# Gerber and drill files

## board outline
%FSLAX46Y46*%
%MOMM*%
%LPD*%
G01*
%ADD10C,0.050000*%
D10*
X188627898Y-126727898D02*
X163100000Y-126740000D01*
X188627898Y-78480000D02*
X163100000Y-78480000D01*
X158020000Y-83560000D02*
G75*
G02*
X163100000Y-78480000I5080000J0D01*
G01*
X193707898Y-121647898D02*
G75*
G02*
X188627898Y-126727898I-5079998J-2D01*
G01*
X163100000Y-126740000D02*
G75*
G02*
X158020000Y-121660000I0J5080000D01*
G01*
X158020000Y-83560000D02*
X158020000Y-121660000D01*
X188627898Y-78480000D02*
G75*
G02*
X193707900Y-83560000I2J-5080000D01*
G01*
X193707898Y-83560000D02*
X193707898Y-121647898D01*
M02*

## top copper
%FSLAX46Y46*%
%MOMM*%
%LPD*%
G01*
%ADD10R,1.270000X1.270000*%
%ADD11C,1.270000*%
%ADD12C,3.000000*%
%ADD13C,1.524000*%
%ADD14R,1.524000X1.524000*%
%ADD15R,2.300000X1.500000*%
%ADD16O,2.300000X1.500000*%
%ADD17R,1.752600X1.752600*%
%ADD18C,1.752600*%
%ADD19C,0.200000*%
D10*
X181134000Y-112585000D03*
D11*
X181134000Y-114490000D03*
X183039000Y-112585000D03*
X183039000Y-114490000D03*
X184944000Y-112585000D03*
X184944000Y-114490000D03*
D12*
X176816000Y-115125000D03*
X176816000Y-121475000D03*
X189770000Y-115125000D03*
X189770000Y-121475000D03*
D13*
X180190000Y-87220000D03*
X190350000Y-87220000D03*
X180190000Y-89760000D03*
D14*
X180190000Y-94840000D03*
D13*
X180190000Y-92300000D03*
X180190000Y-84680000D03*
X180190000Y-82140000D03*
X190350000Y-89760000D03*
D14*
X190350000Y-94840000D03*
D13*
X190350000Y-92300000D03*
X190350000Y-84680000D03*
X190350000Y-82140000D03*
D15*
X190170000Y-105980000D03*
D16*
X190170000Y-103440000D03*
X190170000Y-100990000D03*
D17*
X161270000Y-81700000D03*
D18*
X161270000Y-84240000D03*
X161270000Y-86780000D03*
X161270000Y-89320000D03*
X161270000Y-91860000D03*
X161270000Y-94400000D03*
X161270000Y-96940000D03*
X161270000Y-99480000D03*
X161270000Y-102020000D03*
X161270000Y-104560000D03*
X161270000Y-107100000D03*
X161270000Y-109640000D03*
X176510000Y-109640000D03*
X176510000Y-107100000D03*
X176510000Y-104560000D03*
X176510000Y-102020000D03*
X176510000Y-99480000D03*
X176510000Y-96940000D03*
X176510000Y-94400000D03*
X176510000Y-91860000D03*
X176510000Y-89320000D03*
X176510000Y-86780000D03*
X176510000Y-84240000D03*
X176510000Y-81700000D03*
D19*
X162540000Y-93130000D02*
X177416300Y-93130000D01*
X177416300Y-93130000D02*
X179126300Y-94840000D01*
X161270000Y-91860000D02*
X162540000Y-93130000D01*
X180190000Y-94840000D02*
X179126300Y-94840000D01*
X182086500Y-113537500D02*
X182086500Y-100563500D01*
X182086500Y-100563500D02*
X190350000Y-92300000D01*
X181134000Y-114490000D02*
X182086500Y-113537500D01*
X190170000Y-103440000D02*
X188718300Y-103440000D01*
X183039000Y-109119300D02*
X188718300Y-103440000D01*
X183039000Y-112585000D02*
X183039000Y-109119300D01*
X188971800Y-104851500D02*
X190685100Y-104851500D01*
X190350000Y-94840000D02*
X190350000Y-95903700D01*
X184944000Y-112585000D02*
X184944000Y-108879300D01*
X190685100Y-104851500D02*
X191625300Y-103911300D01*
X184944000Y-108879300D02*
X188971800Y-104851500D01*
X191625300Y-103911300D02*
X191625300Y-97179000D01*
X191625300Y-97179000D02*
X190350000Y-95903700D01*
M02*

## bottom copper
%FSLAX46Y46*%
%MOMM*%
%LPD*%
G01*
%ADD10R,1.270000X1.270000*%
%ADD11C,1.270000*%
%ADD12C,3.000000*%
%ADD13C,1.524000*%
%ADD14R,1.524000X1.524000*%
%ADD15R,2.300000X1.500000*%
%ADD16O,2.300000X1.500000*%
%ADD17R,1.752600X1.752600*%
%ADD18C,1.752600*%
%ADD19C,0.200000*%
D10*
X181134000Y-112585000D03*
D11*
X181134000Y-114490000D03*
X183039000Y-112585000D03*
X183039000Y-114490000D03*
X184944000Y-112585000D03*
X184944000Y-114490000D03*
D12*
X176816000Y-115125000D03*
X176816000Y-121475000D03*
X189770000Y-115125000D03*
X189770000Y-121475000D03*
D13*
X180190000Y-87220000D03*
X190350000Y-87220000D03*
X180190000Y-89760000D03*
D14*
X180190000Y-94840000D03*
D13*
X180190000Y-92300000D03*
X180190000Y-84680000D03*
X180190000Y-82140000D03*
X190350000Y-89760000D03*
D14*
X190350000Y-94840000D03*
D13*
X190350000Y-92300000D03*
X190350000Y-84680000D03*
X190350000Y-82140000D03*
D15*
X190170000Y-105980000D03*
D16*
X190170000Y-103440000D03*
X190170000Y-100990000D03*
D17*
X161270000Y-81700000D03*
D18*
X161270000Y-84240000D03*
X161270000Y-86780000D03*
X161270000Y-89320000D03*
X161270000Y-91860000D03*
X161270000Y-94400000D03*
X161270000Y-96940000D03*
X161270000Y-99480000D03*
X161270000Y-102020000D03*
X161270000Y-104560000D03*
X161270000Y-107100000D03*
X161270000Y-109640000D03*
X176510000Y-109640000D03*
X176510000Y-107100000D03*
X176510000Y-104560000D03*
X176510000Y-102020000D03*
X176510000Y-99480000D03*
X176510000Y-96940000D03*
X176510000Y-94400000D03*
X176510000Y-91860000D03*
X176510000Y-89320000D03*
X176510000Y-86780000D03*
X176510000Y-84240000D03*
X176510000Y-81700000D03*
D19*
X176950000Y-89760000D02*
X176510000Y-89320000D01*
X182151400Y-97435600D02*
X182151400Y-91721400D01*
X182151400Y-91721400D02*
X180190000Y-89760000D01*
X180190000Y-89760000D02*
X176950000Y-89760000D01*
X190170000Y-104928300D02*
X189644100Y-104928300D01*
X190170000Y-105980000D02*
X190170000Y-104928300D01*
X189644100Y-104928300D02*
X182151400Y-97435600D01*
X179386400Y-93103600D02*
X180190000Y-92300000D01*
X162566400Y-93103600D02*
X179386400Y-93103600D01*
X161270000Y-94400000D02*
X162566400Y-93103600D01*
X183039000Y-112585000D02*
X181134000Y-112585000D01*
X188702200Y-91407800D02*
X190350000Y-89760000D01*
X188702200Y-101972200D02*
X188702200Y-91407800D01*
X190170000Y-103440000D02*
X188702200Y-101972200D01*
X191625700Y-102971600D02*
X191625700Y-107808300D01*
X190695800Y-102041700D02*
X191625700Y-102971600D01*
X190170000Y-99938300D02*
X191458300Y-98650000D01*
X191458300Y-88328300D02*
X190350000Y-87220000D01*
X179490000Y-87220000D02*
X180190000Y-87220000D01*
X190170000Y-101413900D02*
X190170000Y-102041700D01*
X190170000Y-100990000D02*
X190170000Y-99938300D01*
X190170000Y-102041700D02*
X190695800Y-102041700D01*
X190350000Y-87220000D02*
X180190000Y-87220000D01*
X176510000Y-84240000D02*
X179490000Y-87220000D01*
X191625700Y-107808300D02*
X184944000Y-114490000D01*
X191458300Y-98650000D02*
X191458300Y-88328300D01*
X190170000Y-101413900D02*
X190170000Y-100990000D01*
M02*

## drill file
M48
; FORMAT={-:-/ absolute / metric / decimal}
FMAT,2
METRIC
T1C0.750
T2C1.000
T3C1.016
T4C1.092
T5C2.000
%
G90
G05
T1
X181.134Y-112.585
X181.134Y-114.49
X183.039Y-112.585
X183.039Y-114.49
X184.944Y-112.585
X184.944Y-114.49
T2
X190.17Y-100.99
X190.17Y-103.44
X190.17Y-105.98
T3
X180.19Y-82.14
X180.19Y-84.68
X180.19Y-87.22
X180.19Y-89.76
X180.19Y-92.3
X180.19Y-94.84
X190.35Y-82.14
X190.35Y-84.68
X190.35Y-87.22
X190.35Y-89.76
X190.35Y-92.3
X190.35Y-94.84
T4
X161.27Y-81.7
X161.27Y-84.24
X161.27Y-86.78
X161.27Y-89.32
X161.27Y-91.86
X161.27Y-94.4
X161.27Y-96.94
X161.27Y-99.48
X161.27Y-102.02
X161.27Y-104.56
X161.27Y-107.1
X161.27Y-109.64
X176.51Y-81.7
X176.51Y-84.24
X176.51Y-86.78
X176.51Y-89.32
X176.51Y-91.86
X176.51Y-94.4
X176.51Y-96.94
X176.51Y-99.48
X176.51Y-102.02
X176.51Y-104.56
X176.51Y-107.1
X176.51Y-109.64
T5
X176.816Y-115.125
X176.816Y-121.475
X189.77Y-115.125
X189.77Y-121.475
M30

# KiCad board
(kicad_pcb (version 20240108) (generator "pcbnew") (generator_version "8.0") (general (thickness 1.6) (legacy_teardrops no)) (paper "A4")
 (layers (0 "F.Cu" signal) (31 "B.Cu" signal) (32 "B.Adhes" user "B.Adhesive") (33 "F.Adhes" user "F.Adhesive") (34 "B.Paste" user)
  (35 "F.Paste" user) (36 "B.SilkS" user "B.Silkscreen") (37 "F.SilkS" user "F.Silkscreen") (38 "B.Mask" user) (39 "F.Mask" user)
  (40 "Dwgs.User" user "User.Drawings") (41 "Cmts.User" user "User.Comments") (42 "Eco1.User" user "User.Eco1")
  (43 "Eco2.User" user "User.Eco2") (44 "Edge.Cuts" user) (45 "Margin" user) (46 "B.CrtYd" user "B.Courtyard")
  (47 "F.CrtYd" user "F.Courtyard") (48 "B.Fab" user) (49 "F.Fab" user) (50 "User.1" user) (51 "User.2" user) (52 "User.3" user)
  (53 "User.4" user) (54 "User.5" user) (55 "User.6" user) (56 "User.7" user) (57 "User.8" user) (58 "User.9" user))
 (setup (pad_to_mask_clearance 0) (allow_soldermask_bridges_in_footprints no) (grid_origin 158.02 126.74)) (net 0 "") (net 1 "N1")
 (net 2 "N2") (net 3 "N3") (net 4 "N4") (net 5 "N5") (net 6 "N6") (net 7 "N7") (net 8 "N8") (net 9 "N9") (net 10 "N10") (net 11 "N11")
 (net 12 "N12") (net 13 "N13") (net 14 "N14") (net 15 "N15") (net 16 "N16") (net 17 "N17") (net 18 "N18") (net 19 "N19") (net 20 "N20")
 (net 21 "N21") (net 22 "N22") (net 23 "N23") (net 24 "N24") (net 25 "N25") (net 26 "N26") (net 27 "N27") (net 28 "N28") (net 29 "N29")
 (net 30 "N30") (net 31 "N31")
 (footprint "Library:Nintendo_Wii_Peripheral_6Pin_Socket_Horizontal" (layer "F.Cu") (at 181.134 112.585)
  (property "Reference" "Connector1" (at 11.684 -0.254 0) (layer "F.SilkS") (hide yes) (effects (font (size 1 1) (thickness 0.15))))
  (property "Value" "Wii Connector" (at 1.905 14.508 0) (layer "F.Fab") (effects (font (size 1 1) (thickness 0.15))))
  (pad "1" thru_hole rect (at 0 0 180) (size 1.27 1.27) (drill 0.75) (layers "*.Cu" "*.Mask") (remove_unused_layers no) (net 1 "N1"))
  (pad "2" thru_hole circle (at 0 1.905 180) (size 1.27 1.27) (drill 0.75) (layers "*.Cu" "*.Mask") (remove_unused_layers no) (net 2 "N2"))
  (pad "3" thru_hole circle (at 1.905 0 180) (size 1.27 1.27) (drill 0.75) (layers "*.Cu" "*.Mask") (remove_unused_layers no) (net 1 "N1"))
  (pad "4" thru_hole circle (at 1.905 1.905 180) (size 1.27 1.27) (drill 0.75) (layers "*.Cu" "*.Mask") (remove_unused_layers no))
  (pad "5" thru_hole circle (at 3.81 0 180) (size 1.27 1.27) (drill 0.75) (layers "*.Cu" "*.Mask") (remove_unused_layers no) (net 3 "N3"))
  (pad "6" thru_hole circle (at 3.81 1.905 180) (size 1.27 1.27) (drill 0.75) (layers "*.Cu" "*.Mask") (remove_unused_layers no)
   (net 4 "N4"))
  (pad "SH" thru_hole circle (at -4.318 2.54 180) (size 3 3) (drill 2) (layers "*.Cu" "*.Mask") (remove_unused_layers no))
  (pad "SH" thru_hole circle (at -4.318 8.89 180) (size 3 3) (drill 2) (layers "*.Cu" "*.Mask") (remove_unused_layers no))
  (pad "SH" thru_hole circle (at 8.636 2.54 180) (size 3 3) (drill 2) (layers "*.Cu" "*.Mask") (remove_unused_layers no))
  (pad "SH" thru_hole circle (at 8.636 8.89 180) (size 3 3) (drill 2) (layers "*.Cu" "*.Mask") (remove_unused_layers no))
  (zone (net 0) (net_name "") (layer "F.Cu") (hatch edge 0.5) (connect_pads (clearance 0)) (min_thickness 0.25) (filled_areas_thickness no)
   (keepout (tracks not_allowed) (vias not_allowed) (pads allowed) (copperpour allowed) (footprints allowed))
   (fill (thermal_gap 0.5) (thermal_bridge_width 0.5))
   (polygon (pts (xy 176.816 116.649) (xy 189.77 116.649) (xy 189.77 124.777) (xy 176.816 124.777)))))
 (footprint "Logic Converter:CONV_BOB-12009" (layer "F.Cu") (at 185.27 88.49 180)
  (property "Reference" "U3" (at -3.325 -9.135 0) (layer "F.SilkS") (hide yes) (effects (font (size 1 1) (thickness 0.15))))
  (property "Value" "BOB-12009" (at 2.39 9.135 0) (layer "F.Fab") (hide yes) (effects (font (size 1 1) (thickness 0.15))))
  (pad "GND_1" thru_hole circle (at 5.08 1.27 180) (size 1.524 1.524) (drill 1.016) (layers "*.Cu" "*.Mask") (remove_unused_layers no)
   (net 4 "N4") (solder_mask_margin 0.102))
  (pad "GND_2" thru_hole circle (at -5.08 1.27 180) (size 1.524 1.524) (drill 1.016) (layers "*.Cu" "*.Mask") (remove_unused_layers no)
   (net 4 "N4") (solder_mask_margin 0.102))
  (pad "HV" thru_hole circle (at 5.08 -1.27 180) (size 1.524 1.524) (drill 1.016) (layers "*.Cu" "*.Mask") (remove_unused_layers no)
   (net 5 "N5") (solder_mask_margin 0.102))
  (pad "HV1" thru_hole rect (at 5.08 -6.35 180) (size 1.524 1.524) (drill 1.016) (layers "*.Cu" "*.Mask") (remove_unused_layers no)
   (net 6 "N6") (solder_mask_margin 0.102))
  (pad "HV2" thru_hole circle (at 5.08 -3.81 180) (size 1.524 1.524) (drill 1.016) (layers "*.Cu" "*.Mask") (remove_unused_layers no)
   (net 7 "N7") (solder_mask_margin 0.102))
  (pad "HV3" thru_hole circle (at 5.08 3.81 180) (size 1.524 1.524) (drill 1.016) (layers "*.Cu" "*.Mask") (remove_unused_layers no)
   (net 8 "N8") (solder_mask_margin 0.102))
  (pad "HV4" thru_hole circle (at 5.08 6.35 180) (size 1.524 1.524) (drill 1.016) (layers "*.Cu" "*.Mask") (remove_unused_layers no)
   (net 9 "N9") (solder_mask_margin 0.102))
  (pad "LV" thru_hole circle (at -5.08 -1.27 180) (size 1.524 1.524) (drill 1.016) (layers "*.Cu" "*.Mask") (remove_unused_layers no)
   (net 1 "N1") (solder_mask_margin 0.102))
  (pad "LV1" thru_hole rect (at -5.08 -6.35 180) (size 1.524 1.524) (drill 1.016) (layers "*.Cu" "*.Mask") (remove_unused_layers no)
   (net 3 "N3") (solder_mask_margin 0.102))
  (pad "LV2" thru_hole circle (at -5.08 -3.81 180) (size 1.524 1.524) (drill 1.016) (layers "*.Cu" "*.Mask") (remove_unused_layers no)
   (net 2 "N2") (solder_mask_margin 0.102))
  (pad "LV3" thru_hole circle (at -5.08 3.81 180) (size 1.524 1.524) (drill 1.016) (layers "*.Cu" "*.Mask") (remove_unused_layers no)
   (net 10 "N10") (solder_mask_margin 0.102))
  (pad "LV4" thru_hole circle (at -5.08 6.35 180) (size 1.524 1.524) (drill 1.016) (layers "*.Cu" "*.Mask") (remove_unused_layers no)
   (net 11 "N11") (solder_mask_margin 0.102)))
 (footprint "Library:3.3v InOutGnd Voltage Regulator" (layer "F.Cu") (at 191.67 103.49 90)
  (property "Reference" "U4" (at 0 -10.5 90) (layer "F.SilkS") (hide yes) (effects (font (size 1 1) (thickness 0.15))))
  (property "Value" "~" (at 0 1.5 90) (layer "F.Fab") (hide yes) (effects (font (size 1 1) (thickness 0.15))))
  (pad "1" thru_hole rect (at -2.49 -1.5 90) (size 1.5 2.3) (drill 1) (layers "*.Cu" "*.Mask") (remove_unused_layers no) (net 5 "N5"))
  (pad "2" thru_hole oval (at 0.05 -1.5 90) (size 1.5 2.3) (drill 1) (layers "*.Cu" "*.Mask") (remove_unused_layers no) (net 1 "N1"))
  (pad "3" thru_hole oval (at 2.5 -1.5 90) (size 1.5 2.3) (drill 1) (layers "*.Cu" "*.Mask") (remove_unused_layers no) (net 4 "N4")))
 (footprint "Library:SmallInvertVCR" (layer "F.Cu") (at 166.77 116.74)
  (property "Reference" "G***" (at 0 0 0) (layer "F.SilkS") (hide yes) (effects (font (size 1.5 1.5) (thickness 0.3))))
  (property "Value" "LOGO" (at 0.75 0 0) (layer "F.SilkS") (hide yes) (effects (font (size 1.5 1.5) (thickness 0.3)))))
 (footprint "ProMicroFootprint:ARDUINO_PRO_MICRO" (layer "F.Cu") (at 168.89 95.67 -90)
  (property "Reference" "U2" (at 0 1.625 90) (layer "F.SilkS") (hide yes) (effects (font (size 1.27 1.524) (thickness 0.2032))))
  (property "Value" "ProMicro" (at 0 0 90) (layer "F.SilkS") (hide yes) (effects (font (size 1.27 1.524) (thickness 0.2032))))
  (pad "1" thru_hole rect (at -13.97 7.62 270) (size 1.7526 1.7526) (drill 1.0922) (layers "*.Cu" "*.SilkS" "*.Mask")
   (remove_unused_layers no) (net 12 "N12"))
  (pad "2" thru_hole circle (at -11.43 7.62 270) (size 1.7526 1.7526) (drill 1.0922) (layers "*.Cu" "*.SilkS" "*.Mask")
   (remove_unused_layers no) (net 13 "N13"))
  (pad "3" thru_hole circle (at -8.89 7.62 270) (size 1.7526 1.7526) (drill 1.0922) (layers "*.Cu" "*.SilkS" "*.Mask")
   (remove_unused_layers no) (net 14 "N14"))
  (pad "4" thru_hole circle (at -6.35 7.62 270) (size 1.7526 1.7526) (drill 1.0922) (layers "*.Cu" "*.SilkS" "*.Mask")
   (remove_unused_layers no) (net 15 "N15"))
  (pad "5" thru_hole circle (at -3.81 7.62 270) (size 1.7526 1.7526) (drill 1.0922) (layers "*.Cu" "*.SilkS" "*.Mask")
   (remove_unused_layers no) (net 6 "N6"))
  (pad "6" thru_hole circle (at -1.27 7.62 270) (size 1.7526 1.7526) (drill 1.0922) (layers "*.Cu" "*.SilkS" "*.Mask")
   (remove_unused_layers no) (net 7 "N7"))
  (pad "7" thru_hole circle (at 1.27 7.62 270) (size 1.7526 1.7526) (drill 1.0922) (layers "*.Cu" "*.SilkS" "*.Mask")
   (remove_unused_layers no) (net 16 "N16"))
  (pad "8" thru_hole circle (at 3.81 7.62 270) (size 1.7526 1.7526) (drill 1.0922) (layers "*.Cu" "*.SilkS" "*.Mask")
   (remove_unused_layers no) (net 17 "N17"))
  (pad "9" thru_hole circle (at 6.35 7.62 270) (size 1.7526 1.7526) (drill 1.0922) (layers "*.Cu" "*.SilkS" "*.Mask")
   (remove_unused_layers no) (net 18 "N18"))
  (pad "10" thru_hole circle (at 8.89 7.62 270) (size 1.7526 1.7526) (drill 1.0922) (layers "*.Cu" "*.SilkS" "*.Mask")
   (remove_unused_layers no) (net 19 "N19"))
  (pad "11" thru_hole circle (at 11.43 7.62 270) (size 1.7526 1.7526) (drill 1.0922) (layers "*.Cu" "*.SilkS" "*.Mask")
   (remove_unused_layers no) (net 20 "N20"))
  (pad "12" thru_hole circle (at 13.97 7.62 270) (size 1.7526 1.7526) (drill 1.0922) (layers "*.Cu" "*.SilkS" "*.Mask")
   (remove_unused_layers no) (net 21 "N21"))
  (pad "13" thru_hole circle (at 13.97 -7.62 270) (size 1.7526 1.7526) (drill 1.0922) (layers "*.Cu" "*.SilkS" "*.Mask")
   (remove_unused_layers no) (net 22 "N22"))
  (pad "14" thru_hole circle (at 11.43 -7.62 270) (size 1.7526 1.7526) (drill 1.0922) (layers "*.Cu" "*.SilkS" "*.Mask")
   (remove_unused_layers no) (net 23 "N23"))
  (pad "15" thru_hole circle (at 8.89 -7.62 270) (size 1.7526 1.7526) (drill 1.0922) (layers "*.Cu" "*.SilkS" "*.Mask")
   (remove_unused_layers no) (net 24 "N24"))
  (pad "16" thru_hole circle (at 6.35 -7.62 270) (size 1.7526 1.7526) (drill 1.0922) (layers "*.Cu" "*.SilkS" "*.Mask")
   (remove_unused_layers no) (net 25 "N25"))
  (pad "17" thru_hole circle (at 3.81 -7.62 270) (size 1.7526 1.7526) (drill 1.0922) (layers "*.Cu" "*.SilkS" "*.Mask")
   (remove_unused_layers no) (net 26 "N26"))
  (pad "18" thru_hole circle (at 1.27 -7.62 270) (size 1.7526 1.7526) (drill 1.0922) (layers "*.Cu" "*.SilkS" "*.Mask")
   (remove_unused_layers no) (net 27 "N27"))
  (pad "19" thru_hole circle (at -1.27 -7.62 270) (size 1.7526 1.7526) (drill 1.0922) (layers "*.Cu" "*.SilkS" "*.Mask")
   (remove_unused_layers no) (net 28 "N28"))
  (pad "20" thru_hole circle (at -3.81 -7.62 270) (size 1.7526 1.7526) (drill 1.0922) (layers "*.Cu" "*.SilkS" "*.Mask")
   (remove_unused_layers no) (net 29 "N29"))
  (pad "21" thru_hole circle (at -6.35 -7.62 270) (size 1.7526 1.7526) (drill 1.0922) (layers "*.Cu" "*.SilkS" "*.Mask")
   (remove_unused_layers no) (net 5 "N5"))
  (pad "22" thru_hole circle (at -8.89 -7.62 270) (size 1.7526 1.7526) (drill 1.0922) (layers "*.Cu" "*.SilkS" "*.Mask")
   (remove_unused_layers no) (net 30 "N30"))
  (pad "23" thru_hole circle (at -11.43 -7.62 270) (size 1.7526 1.7526) (drill 1.0922) (layers "*.Cu" "*.SilkS" "*.Mask")
   (remove_unused_layers no) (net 4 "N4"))
  (pad "24" thru_hole circle (at -13.97 -7.62 270) (size 1.7526 1.7526) (drill 1.0922) (layers "*.Cu" "*.SilkS" "*.Mask")
   (remove_unused_layers no) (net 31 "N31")))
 (gr_line (start 188.627898 126.727898) (end 163.1 126.74) (stroke (width 0.05) (type default)) (layer "Edge.Cuts"))
 (gr_line (start 188.627898 78.48) (end 163.1 78.48) (stroke (width 0.05) (type default)) (layer "Edge.Cuts"))
 (gr_arc (start 158.02 83.56) (mid 159.507898 79.967898) (end 163.1 78.48) (stroke (width 0.05) (type default)) (layer "Edge.Cuts"))
 (gr_arc (start 193.707898 121.647898) (mid 192.22 125.24) (end 188.627898 126.727898) (stroke (width 0.05) (type default))
  (layer "Edge.Cuts"))
 (gr_arc (start 163.1 126.74) (mid 159.507898 125.252102) (end 158.02 121.66) (stroke (width 0.05) (type default)) (layer "Edge.Cuts"))
 (gr_line (start 158.02 83.56) (end 158.02 121.66) (stroke (width 0.05) (type default)) (layer "Edge.Cuts"))
 (gr_arc (start 188.627898 78.48) (mid 192.22 79.967898) (end 193.707898 83.56) (stroke (width 0.05) (type default)) (layer "Edge.Cuts"))
 (gr_line (start 193.707898 83.56) (end 193.707898 121.647898) (stroke (width 0.05) (type default)) (layer "Edge.Cuts"))
 (segment (start 162.54 93.13) (end 177.4163 93.13) (width 0.2) (layer "F.Cu") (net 6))
 (segment (start 177.4163 93.13) (end 179.1263 94.84) (width 0.2) (layer "F.Cu") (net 6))
 (segment (start 161.27 91.86) (end 162.54 93.13) (width 0.2) (layer "F.Cu") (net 6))
 (segment (start 180.19 94.84) (end 179.1263 94.84) (width 0.2) (layer "F.Cu") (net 6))
 (segment (start 176.95 89.76) (end 176.51 89.32) (width 0.2) (layer "B.Cu") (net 5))
 (segment (start 182.1514 97.4356) (end 182.1514 91.7214) (width 0.2) (layer "B.Cu") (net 5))
 (segment (start 182.1514 91.7214) (end 180.19 89.76) (width 0.2) (layer "B.Cu") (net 5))
 (segment (start 180.19 89.76) (end 176.95 89.76) (width 0.2) (layer "B.Cu") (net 5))
 (segment (start 190.17 104.9283) (end 189.6441 104.9283) (width 0.2) (layer "B.Cu") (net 5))
 (segment (start 190.17 105.98) (end 190.17 104.9283) (width 0.2) (layer "B.Cu") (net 5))
 (segment (start 189.6441 104.9283) (end 182.1514 97.4356) (width 0.2) (layer "B.Cu") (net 5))
 (segment (start 179.3864 93.1036) (end 180.19 92.3) (width 0.2) (layer "B.Cu") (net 7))
 (segment (start 162.5664 93.1036) (end 179.3864 93.1036) (width 0.2) (layer "B.Cu") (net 7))
 (segment (start 161.27 94.4) (end 162.5664 93.1036) (width 0.2) (layer "B.Cu") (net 7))
 (segment (start 182.0865 113.5375) (end 182.0865 100.5635) (width 0.2) (layer "F.Cu") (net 2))
 (segment (start 182.0865 100.5635) (end 190.35 92.3) (width 0.2) (layer "F.Cu") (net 2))
 (segment (start 181.134 114.49) (end 182.0865 113.5375) (width 0.2) (layer "F.Cu") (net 2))
 (segment (start 190.17 103.44) (end 188.7183 103.44) (width 0.2) (layer "F.Cu") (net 1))
 (segment (start 183.039 109.1193) (end 188.7183 103.44) (width 0.2) (layer "F.Cu") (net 1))
 (segment (start 183.039 112.585) (end 183.039 109.1193) (width 0.2) (layer "F.Cu") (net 1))
 (segment (start 183.039 112.585) (end 181.134 112.585) (width 0.2) (layer "B.Cu") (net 1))
 (segment (start 188.7022 91.4078) (end 190.35 89.76) (width 0.2) (layer "B.Cu") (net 1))
 (segment (start 188.7022 101.9722) (end 188.7022 91.4078) (width 0.2) (layer "B.Cu") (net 1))
 (segment (start 190.17 103.44) (end 188.7022 101.9722) (width 0.2) (layer "B.Cu") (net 1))
 (segment (start 188.9718 104.8515) (end 190.6851 104.8515) (width 0.2) (layer "F.Cu") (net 3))
 (segment (start 190.35 94.84) (end 190.35 95.9037) (width 0.2) (layer "F.Cu") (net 3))
 (segment (start 184.944 112.585) (end 184.944 108.8793) (width 0.2) (layer "F.Cu") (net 3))
 (segment (start 190.6851 104.8515) (end 191.6253 103.9113) (width 0.2) (layer "F.Cu") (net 3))
 (segment (start 184.944 108.8793) (end 188.9718 104.8515) (width 0.2) (layer "F.Cu") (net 3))
 (segment (start 191.6253 103.9113) (end 191.6253 97.179) (width 0.2) (layer "F.Cu") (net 3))
 (segment (start 191.6253 97.179) (end 190.35 95.9037) (width 0.2) (layer "F.Cu") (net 3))
 (segment (start 191.6257 102.9716) (end 191.6257 107.8083) (width 0.2) (layer "B.Cu") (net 4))
 (segment (start 190.6958 102.0417) (end 191.6257 102.9716) (width 0.2) (layer "B.Cu") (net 4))
 (segment (start 190.17 99.9383) (end 191.4583 98.65) (width 0.2) (layer "B.Cu") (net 4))
 (segment (start 191.4583 88.3283) (end 190.35 87.22) (width 0.2) (layer "B.Cu") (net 4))
 (segment (start 179.49 87.22) (end 180.19 87.22) (width 0.2) (layer "B.Cu") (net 4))
 (segment (start 190.17 101.4139) (end 190.17 102.0417) (width 0.2) (layer "B.Cu") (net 4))
 (segment (start 190.17 100.99) (end 190.17 99.9383) (width 0.2) (layer "B.Cu") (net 4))
 (segment (start 190.17 102.0417) (end 190.6958 102.0417) (width 0.2) (layer "B.Cu") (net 4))
 (segment (start 190.35 87.22) (end 180.19 87.22) (width 0.2) (layer "B.Cu") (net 4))
 (segment (start 176.51 84.24) (end 179.49 87.22) (width 0.2) (layer "B.Cu") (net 4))
 (segment (start 191.6257 107.8083) (end 184.944 114.49) (width 0.2) (layer "B.Cu") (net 4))
 (segment (start 191.4583 98.65) (end 191.4583 88.3283) (width 0.2) (layer "B.Cu") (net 4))
 (segment (start 190.17 101.4139) (end 190.17 100.99) (width 0.2) (layer "B.Cu") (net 4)))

